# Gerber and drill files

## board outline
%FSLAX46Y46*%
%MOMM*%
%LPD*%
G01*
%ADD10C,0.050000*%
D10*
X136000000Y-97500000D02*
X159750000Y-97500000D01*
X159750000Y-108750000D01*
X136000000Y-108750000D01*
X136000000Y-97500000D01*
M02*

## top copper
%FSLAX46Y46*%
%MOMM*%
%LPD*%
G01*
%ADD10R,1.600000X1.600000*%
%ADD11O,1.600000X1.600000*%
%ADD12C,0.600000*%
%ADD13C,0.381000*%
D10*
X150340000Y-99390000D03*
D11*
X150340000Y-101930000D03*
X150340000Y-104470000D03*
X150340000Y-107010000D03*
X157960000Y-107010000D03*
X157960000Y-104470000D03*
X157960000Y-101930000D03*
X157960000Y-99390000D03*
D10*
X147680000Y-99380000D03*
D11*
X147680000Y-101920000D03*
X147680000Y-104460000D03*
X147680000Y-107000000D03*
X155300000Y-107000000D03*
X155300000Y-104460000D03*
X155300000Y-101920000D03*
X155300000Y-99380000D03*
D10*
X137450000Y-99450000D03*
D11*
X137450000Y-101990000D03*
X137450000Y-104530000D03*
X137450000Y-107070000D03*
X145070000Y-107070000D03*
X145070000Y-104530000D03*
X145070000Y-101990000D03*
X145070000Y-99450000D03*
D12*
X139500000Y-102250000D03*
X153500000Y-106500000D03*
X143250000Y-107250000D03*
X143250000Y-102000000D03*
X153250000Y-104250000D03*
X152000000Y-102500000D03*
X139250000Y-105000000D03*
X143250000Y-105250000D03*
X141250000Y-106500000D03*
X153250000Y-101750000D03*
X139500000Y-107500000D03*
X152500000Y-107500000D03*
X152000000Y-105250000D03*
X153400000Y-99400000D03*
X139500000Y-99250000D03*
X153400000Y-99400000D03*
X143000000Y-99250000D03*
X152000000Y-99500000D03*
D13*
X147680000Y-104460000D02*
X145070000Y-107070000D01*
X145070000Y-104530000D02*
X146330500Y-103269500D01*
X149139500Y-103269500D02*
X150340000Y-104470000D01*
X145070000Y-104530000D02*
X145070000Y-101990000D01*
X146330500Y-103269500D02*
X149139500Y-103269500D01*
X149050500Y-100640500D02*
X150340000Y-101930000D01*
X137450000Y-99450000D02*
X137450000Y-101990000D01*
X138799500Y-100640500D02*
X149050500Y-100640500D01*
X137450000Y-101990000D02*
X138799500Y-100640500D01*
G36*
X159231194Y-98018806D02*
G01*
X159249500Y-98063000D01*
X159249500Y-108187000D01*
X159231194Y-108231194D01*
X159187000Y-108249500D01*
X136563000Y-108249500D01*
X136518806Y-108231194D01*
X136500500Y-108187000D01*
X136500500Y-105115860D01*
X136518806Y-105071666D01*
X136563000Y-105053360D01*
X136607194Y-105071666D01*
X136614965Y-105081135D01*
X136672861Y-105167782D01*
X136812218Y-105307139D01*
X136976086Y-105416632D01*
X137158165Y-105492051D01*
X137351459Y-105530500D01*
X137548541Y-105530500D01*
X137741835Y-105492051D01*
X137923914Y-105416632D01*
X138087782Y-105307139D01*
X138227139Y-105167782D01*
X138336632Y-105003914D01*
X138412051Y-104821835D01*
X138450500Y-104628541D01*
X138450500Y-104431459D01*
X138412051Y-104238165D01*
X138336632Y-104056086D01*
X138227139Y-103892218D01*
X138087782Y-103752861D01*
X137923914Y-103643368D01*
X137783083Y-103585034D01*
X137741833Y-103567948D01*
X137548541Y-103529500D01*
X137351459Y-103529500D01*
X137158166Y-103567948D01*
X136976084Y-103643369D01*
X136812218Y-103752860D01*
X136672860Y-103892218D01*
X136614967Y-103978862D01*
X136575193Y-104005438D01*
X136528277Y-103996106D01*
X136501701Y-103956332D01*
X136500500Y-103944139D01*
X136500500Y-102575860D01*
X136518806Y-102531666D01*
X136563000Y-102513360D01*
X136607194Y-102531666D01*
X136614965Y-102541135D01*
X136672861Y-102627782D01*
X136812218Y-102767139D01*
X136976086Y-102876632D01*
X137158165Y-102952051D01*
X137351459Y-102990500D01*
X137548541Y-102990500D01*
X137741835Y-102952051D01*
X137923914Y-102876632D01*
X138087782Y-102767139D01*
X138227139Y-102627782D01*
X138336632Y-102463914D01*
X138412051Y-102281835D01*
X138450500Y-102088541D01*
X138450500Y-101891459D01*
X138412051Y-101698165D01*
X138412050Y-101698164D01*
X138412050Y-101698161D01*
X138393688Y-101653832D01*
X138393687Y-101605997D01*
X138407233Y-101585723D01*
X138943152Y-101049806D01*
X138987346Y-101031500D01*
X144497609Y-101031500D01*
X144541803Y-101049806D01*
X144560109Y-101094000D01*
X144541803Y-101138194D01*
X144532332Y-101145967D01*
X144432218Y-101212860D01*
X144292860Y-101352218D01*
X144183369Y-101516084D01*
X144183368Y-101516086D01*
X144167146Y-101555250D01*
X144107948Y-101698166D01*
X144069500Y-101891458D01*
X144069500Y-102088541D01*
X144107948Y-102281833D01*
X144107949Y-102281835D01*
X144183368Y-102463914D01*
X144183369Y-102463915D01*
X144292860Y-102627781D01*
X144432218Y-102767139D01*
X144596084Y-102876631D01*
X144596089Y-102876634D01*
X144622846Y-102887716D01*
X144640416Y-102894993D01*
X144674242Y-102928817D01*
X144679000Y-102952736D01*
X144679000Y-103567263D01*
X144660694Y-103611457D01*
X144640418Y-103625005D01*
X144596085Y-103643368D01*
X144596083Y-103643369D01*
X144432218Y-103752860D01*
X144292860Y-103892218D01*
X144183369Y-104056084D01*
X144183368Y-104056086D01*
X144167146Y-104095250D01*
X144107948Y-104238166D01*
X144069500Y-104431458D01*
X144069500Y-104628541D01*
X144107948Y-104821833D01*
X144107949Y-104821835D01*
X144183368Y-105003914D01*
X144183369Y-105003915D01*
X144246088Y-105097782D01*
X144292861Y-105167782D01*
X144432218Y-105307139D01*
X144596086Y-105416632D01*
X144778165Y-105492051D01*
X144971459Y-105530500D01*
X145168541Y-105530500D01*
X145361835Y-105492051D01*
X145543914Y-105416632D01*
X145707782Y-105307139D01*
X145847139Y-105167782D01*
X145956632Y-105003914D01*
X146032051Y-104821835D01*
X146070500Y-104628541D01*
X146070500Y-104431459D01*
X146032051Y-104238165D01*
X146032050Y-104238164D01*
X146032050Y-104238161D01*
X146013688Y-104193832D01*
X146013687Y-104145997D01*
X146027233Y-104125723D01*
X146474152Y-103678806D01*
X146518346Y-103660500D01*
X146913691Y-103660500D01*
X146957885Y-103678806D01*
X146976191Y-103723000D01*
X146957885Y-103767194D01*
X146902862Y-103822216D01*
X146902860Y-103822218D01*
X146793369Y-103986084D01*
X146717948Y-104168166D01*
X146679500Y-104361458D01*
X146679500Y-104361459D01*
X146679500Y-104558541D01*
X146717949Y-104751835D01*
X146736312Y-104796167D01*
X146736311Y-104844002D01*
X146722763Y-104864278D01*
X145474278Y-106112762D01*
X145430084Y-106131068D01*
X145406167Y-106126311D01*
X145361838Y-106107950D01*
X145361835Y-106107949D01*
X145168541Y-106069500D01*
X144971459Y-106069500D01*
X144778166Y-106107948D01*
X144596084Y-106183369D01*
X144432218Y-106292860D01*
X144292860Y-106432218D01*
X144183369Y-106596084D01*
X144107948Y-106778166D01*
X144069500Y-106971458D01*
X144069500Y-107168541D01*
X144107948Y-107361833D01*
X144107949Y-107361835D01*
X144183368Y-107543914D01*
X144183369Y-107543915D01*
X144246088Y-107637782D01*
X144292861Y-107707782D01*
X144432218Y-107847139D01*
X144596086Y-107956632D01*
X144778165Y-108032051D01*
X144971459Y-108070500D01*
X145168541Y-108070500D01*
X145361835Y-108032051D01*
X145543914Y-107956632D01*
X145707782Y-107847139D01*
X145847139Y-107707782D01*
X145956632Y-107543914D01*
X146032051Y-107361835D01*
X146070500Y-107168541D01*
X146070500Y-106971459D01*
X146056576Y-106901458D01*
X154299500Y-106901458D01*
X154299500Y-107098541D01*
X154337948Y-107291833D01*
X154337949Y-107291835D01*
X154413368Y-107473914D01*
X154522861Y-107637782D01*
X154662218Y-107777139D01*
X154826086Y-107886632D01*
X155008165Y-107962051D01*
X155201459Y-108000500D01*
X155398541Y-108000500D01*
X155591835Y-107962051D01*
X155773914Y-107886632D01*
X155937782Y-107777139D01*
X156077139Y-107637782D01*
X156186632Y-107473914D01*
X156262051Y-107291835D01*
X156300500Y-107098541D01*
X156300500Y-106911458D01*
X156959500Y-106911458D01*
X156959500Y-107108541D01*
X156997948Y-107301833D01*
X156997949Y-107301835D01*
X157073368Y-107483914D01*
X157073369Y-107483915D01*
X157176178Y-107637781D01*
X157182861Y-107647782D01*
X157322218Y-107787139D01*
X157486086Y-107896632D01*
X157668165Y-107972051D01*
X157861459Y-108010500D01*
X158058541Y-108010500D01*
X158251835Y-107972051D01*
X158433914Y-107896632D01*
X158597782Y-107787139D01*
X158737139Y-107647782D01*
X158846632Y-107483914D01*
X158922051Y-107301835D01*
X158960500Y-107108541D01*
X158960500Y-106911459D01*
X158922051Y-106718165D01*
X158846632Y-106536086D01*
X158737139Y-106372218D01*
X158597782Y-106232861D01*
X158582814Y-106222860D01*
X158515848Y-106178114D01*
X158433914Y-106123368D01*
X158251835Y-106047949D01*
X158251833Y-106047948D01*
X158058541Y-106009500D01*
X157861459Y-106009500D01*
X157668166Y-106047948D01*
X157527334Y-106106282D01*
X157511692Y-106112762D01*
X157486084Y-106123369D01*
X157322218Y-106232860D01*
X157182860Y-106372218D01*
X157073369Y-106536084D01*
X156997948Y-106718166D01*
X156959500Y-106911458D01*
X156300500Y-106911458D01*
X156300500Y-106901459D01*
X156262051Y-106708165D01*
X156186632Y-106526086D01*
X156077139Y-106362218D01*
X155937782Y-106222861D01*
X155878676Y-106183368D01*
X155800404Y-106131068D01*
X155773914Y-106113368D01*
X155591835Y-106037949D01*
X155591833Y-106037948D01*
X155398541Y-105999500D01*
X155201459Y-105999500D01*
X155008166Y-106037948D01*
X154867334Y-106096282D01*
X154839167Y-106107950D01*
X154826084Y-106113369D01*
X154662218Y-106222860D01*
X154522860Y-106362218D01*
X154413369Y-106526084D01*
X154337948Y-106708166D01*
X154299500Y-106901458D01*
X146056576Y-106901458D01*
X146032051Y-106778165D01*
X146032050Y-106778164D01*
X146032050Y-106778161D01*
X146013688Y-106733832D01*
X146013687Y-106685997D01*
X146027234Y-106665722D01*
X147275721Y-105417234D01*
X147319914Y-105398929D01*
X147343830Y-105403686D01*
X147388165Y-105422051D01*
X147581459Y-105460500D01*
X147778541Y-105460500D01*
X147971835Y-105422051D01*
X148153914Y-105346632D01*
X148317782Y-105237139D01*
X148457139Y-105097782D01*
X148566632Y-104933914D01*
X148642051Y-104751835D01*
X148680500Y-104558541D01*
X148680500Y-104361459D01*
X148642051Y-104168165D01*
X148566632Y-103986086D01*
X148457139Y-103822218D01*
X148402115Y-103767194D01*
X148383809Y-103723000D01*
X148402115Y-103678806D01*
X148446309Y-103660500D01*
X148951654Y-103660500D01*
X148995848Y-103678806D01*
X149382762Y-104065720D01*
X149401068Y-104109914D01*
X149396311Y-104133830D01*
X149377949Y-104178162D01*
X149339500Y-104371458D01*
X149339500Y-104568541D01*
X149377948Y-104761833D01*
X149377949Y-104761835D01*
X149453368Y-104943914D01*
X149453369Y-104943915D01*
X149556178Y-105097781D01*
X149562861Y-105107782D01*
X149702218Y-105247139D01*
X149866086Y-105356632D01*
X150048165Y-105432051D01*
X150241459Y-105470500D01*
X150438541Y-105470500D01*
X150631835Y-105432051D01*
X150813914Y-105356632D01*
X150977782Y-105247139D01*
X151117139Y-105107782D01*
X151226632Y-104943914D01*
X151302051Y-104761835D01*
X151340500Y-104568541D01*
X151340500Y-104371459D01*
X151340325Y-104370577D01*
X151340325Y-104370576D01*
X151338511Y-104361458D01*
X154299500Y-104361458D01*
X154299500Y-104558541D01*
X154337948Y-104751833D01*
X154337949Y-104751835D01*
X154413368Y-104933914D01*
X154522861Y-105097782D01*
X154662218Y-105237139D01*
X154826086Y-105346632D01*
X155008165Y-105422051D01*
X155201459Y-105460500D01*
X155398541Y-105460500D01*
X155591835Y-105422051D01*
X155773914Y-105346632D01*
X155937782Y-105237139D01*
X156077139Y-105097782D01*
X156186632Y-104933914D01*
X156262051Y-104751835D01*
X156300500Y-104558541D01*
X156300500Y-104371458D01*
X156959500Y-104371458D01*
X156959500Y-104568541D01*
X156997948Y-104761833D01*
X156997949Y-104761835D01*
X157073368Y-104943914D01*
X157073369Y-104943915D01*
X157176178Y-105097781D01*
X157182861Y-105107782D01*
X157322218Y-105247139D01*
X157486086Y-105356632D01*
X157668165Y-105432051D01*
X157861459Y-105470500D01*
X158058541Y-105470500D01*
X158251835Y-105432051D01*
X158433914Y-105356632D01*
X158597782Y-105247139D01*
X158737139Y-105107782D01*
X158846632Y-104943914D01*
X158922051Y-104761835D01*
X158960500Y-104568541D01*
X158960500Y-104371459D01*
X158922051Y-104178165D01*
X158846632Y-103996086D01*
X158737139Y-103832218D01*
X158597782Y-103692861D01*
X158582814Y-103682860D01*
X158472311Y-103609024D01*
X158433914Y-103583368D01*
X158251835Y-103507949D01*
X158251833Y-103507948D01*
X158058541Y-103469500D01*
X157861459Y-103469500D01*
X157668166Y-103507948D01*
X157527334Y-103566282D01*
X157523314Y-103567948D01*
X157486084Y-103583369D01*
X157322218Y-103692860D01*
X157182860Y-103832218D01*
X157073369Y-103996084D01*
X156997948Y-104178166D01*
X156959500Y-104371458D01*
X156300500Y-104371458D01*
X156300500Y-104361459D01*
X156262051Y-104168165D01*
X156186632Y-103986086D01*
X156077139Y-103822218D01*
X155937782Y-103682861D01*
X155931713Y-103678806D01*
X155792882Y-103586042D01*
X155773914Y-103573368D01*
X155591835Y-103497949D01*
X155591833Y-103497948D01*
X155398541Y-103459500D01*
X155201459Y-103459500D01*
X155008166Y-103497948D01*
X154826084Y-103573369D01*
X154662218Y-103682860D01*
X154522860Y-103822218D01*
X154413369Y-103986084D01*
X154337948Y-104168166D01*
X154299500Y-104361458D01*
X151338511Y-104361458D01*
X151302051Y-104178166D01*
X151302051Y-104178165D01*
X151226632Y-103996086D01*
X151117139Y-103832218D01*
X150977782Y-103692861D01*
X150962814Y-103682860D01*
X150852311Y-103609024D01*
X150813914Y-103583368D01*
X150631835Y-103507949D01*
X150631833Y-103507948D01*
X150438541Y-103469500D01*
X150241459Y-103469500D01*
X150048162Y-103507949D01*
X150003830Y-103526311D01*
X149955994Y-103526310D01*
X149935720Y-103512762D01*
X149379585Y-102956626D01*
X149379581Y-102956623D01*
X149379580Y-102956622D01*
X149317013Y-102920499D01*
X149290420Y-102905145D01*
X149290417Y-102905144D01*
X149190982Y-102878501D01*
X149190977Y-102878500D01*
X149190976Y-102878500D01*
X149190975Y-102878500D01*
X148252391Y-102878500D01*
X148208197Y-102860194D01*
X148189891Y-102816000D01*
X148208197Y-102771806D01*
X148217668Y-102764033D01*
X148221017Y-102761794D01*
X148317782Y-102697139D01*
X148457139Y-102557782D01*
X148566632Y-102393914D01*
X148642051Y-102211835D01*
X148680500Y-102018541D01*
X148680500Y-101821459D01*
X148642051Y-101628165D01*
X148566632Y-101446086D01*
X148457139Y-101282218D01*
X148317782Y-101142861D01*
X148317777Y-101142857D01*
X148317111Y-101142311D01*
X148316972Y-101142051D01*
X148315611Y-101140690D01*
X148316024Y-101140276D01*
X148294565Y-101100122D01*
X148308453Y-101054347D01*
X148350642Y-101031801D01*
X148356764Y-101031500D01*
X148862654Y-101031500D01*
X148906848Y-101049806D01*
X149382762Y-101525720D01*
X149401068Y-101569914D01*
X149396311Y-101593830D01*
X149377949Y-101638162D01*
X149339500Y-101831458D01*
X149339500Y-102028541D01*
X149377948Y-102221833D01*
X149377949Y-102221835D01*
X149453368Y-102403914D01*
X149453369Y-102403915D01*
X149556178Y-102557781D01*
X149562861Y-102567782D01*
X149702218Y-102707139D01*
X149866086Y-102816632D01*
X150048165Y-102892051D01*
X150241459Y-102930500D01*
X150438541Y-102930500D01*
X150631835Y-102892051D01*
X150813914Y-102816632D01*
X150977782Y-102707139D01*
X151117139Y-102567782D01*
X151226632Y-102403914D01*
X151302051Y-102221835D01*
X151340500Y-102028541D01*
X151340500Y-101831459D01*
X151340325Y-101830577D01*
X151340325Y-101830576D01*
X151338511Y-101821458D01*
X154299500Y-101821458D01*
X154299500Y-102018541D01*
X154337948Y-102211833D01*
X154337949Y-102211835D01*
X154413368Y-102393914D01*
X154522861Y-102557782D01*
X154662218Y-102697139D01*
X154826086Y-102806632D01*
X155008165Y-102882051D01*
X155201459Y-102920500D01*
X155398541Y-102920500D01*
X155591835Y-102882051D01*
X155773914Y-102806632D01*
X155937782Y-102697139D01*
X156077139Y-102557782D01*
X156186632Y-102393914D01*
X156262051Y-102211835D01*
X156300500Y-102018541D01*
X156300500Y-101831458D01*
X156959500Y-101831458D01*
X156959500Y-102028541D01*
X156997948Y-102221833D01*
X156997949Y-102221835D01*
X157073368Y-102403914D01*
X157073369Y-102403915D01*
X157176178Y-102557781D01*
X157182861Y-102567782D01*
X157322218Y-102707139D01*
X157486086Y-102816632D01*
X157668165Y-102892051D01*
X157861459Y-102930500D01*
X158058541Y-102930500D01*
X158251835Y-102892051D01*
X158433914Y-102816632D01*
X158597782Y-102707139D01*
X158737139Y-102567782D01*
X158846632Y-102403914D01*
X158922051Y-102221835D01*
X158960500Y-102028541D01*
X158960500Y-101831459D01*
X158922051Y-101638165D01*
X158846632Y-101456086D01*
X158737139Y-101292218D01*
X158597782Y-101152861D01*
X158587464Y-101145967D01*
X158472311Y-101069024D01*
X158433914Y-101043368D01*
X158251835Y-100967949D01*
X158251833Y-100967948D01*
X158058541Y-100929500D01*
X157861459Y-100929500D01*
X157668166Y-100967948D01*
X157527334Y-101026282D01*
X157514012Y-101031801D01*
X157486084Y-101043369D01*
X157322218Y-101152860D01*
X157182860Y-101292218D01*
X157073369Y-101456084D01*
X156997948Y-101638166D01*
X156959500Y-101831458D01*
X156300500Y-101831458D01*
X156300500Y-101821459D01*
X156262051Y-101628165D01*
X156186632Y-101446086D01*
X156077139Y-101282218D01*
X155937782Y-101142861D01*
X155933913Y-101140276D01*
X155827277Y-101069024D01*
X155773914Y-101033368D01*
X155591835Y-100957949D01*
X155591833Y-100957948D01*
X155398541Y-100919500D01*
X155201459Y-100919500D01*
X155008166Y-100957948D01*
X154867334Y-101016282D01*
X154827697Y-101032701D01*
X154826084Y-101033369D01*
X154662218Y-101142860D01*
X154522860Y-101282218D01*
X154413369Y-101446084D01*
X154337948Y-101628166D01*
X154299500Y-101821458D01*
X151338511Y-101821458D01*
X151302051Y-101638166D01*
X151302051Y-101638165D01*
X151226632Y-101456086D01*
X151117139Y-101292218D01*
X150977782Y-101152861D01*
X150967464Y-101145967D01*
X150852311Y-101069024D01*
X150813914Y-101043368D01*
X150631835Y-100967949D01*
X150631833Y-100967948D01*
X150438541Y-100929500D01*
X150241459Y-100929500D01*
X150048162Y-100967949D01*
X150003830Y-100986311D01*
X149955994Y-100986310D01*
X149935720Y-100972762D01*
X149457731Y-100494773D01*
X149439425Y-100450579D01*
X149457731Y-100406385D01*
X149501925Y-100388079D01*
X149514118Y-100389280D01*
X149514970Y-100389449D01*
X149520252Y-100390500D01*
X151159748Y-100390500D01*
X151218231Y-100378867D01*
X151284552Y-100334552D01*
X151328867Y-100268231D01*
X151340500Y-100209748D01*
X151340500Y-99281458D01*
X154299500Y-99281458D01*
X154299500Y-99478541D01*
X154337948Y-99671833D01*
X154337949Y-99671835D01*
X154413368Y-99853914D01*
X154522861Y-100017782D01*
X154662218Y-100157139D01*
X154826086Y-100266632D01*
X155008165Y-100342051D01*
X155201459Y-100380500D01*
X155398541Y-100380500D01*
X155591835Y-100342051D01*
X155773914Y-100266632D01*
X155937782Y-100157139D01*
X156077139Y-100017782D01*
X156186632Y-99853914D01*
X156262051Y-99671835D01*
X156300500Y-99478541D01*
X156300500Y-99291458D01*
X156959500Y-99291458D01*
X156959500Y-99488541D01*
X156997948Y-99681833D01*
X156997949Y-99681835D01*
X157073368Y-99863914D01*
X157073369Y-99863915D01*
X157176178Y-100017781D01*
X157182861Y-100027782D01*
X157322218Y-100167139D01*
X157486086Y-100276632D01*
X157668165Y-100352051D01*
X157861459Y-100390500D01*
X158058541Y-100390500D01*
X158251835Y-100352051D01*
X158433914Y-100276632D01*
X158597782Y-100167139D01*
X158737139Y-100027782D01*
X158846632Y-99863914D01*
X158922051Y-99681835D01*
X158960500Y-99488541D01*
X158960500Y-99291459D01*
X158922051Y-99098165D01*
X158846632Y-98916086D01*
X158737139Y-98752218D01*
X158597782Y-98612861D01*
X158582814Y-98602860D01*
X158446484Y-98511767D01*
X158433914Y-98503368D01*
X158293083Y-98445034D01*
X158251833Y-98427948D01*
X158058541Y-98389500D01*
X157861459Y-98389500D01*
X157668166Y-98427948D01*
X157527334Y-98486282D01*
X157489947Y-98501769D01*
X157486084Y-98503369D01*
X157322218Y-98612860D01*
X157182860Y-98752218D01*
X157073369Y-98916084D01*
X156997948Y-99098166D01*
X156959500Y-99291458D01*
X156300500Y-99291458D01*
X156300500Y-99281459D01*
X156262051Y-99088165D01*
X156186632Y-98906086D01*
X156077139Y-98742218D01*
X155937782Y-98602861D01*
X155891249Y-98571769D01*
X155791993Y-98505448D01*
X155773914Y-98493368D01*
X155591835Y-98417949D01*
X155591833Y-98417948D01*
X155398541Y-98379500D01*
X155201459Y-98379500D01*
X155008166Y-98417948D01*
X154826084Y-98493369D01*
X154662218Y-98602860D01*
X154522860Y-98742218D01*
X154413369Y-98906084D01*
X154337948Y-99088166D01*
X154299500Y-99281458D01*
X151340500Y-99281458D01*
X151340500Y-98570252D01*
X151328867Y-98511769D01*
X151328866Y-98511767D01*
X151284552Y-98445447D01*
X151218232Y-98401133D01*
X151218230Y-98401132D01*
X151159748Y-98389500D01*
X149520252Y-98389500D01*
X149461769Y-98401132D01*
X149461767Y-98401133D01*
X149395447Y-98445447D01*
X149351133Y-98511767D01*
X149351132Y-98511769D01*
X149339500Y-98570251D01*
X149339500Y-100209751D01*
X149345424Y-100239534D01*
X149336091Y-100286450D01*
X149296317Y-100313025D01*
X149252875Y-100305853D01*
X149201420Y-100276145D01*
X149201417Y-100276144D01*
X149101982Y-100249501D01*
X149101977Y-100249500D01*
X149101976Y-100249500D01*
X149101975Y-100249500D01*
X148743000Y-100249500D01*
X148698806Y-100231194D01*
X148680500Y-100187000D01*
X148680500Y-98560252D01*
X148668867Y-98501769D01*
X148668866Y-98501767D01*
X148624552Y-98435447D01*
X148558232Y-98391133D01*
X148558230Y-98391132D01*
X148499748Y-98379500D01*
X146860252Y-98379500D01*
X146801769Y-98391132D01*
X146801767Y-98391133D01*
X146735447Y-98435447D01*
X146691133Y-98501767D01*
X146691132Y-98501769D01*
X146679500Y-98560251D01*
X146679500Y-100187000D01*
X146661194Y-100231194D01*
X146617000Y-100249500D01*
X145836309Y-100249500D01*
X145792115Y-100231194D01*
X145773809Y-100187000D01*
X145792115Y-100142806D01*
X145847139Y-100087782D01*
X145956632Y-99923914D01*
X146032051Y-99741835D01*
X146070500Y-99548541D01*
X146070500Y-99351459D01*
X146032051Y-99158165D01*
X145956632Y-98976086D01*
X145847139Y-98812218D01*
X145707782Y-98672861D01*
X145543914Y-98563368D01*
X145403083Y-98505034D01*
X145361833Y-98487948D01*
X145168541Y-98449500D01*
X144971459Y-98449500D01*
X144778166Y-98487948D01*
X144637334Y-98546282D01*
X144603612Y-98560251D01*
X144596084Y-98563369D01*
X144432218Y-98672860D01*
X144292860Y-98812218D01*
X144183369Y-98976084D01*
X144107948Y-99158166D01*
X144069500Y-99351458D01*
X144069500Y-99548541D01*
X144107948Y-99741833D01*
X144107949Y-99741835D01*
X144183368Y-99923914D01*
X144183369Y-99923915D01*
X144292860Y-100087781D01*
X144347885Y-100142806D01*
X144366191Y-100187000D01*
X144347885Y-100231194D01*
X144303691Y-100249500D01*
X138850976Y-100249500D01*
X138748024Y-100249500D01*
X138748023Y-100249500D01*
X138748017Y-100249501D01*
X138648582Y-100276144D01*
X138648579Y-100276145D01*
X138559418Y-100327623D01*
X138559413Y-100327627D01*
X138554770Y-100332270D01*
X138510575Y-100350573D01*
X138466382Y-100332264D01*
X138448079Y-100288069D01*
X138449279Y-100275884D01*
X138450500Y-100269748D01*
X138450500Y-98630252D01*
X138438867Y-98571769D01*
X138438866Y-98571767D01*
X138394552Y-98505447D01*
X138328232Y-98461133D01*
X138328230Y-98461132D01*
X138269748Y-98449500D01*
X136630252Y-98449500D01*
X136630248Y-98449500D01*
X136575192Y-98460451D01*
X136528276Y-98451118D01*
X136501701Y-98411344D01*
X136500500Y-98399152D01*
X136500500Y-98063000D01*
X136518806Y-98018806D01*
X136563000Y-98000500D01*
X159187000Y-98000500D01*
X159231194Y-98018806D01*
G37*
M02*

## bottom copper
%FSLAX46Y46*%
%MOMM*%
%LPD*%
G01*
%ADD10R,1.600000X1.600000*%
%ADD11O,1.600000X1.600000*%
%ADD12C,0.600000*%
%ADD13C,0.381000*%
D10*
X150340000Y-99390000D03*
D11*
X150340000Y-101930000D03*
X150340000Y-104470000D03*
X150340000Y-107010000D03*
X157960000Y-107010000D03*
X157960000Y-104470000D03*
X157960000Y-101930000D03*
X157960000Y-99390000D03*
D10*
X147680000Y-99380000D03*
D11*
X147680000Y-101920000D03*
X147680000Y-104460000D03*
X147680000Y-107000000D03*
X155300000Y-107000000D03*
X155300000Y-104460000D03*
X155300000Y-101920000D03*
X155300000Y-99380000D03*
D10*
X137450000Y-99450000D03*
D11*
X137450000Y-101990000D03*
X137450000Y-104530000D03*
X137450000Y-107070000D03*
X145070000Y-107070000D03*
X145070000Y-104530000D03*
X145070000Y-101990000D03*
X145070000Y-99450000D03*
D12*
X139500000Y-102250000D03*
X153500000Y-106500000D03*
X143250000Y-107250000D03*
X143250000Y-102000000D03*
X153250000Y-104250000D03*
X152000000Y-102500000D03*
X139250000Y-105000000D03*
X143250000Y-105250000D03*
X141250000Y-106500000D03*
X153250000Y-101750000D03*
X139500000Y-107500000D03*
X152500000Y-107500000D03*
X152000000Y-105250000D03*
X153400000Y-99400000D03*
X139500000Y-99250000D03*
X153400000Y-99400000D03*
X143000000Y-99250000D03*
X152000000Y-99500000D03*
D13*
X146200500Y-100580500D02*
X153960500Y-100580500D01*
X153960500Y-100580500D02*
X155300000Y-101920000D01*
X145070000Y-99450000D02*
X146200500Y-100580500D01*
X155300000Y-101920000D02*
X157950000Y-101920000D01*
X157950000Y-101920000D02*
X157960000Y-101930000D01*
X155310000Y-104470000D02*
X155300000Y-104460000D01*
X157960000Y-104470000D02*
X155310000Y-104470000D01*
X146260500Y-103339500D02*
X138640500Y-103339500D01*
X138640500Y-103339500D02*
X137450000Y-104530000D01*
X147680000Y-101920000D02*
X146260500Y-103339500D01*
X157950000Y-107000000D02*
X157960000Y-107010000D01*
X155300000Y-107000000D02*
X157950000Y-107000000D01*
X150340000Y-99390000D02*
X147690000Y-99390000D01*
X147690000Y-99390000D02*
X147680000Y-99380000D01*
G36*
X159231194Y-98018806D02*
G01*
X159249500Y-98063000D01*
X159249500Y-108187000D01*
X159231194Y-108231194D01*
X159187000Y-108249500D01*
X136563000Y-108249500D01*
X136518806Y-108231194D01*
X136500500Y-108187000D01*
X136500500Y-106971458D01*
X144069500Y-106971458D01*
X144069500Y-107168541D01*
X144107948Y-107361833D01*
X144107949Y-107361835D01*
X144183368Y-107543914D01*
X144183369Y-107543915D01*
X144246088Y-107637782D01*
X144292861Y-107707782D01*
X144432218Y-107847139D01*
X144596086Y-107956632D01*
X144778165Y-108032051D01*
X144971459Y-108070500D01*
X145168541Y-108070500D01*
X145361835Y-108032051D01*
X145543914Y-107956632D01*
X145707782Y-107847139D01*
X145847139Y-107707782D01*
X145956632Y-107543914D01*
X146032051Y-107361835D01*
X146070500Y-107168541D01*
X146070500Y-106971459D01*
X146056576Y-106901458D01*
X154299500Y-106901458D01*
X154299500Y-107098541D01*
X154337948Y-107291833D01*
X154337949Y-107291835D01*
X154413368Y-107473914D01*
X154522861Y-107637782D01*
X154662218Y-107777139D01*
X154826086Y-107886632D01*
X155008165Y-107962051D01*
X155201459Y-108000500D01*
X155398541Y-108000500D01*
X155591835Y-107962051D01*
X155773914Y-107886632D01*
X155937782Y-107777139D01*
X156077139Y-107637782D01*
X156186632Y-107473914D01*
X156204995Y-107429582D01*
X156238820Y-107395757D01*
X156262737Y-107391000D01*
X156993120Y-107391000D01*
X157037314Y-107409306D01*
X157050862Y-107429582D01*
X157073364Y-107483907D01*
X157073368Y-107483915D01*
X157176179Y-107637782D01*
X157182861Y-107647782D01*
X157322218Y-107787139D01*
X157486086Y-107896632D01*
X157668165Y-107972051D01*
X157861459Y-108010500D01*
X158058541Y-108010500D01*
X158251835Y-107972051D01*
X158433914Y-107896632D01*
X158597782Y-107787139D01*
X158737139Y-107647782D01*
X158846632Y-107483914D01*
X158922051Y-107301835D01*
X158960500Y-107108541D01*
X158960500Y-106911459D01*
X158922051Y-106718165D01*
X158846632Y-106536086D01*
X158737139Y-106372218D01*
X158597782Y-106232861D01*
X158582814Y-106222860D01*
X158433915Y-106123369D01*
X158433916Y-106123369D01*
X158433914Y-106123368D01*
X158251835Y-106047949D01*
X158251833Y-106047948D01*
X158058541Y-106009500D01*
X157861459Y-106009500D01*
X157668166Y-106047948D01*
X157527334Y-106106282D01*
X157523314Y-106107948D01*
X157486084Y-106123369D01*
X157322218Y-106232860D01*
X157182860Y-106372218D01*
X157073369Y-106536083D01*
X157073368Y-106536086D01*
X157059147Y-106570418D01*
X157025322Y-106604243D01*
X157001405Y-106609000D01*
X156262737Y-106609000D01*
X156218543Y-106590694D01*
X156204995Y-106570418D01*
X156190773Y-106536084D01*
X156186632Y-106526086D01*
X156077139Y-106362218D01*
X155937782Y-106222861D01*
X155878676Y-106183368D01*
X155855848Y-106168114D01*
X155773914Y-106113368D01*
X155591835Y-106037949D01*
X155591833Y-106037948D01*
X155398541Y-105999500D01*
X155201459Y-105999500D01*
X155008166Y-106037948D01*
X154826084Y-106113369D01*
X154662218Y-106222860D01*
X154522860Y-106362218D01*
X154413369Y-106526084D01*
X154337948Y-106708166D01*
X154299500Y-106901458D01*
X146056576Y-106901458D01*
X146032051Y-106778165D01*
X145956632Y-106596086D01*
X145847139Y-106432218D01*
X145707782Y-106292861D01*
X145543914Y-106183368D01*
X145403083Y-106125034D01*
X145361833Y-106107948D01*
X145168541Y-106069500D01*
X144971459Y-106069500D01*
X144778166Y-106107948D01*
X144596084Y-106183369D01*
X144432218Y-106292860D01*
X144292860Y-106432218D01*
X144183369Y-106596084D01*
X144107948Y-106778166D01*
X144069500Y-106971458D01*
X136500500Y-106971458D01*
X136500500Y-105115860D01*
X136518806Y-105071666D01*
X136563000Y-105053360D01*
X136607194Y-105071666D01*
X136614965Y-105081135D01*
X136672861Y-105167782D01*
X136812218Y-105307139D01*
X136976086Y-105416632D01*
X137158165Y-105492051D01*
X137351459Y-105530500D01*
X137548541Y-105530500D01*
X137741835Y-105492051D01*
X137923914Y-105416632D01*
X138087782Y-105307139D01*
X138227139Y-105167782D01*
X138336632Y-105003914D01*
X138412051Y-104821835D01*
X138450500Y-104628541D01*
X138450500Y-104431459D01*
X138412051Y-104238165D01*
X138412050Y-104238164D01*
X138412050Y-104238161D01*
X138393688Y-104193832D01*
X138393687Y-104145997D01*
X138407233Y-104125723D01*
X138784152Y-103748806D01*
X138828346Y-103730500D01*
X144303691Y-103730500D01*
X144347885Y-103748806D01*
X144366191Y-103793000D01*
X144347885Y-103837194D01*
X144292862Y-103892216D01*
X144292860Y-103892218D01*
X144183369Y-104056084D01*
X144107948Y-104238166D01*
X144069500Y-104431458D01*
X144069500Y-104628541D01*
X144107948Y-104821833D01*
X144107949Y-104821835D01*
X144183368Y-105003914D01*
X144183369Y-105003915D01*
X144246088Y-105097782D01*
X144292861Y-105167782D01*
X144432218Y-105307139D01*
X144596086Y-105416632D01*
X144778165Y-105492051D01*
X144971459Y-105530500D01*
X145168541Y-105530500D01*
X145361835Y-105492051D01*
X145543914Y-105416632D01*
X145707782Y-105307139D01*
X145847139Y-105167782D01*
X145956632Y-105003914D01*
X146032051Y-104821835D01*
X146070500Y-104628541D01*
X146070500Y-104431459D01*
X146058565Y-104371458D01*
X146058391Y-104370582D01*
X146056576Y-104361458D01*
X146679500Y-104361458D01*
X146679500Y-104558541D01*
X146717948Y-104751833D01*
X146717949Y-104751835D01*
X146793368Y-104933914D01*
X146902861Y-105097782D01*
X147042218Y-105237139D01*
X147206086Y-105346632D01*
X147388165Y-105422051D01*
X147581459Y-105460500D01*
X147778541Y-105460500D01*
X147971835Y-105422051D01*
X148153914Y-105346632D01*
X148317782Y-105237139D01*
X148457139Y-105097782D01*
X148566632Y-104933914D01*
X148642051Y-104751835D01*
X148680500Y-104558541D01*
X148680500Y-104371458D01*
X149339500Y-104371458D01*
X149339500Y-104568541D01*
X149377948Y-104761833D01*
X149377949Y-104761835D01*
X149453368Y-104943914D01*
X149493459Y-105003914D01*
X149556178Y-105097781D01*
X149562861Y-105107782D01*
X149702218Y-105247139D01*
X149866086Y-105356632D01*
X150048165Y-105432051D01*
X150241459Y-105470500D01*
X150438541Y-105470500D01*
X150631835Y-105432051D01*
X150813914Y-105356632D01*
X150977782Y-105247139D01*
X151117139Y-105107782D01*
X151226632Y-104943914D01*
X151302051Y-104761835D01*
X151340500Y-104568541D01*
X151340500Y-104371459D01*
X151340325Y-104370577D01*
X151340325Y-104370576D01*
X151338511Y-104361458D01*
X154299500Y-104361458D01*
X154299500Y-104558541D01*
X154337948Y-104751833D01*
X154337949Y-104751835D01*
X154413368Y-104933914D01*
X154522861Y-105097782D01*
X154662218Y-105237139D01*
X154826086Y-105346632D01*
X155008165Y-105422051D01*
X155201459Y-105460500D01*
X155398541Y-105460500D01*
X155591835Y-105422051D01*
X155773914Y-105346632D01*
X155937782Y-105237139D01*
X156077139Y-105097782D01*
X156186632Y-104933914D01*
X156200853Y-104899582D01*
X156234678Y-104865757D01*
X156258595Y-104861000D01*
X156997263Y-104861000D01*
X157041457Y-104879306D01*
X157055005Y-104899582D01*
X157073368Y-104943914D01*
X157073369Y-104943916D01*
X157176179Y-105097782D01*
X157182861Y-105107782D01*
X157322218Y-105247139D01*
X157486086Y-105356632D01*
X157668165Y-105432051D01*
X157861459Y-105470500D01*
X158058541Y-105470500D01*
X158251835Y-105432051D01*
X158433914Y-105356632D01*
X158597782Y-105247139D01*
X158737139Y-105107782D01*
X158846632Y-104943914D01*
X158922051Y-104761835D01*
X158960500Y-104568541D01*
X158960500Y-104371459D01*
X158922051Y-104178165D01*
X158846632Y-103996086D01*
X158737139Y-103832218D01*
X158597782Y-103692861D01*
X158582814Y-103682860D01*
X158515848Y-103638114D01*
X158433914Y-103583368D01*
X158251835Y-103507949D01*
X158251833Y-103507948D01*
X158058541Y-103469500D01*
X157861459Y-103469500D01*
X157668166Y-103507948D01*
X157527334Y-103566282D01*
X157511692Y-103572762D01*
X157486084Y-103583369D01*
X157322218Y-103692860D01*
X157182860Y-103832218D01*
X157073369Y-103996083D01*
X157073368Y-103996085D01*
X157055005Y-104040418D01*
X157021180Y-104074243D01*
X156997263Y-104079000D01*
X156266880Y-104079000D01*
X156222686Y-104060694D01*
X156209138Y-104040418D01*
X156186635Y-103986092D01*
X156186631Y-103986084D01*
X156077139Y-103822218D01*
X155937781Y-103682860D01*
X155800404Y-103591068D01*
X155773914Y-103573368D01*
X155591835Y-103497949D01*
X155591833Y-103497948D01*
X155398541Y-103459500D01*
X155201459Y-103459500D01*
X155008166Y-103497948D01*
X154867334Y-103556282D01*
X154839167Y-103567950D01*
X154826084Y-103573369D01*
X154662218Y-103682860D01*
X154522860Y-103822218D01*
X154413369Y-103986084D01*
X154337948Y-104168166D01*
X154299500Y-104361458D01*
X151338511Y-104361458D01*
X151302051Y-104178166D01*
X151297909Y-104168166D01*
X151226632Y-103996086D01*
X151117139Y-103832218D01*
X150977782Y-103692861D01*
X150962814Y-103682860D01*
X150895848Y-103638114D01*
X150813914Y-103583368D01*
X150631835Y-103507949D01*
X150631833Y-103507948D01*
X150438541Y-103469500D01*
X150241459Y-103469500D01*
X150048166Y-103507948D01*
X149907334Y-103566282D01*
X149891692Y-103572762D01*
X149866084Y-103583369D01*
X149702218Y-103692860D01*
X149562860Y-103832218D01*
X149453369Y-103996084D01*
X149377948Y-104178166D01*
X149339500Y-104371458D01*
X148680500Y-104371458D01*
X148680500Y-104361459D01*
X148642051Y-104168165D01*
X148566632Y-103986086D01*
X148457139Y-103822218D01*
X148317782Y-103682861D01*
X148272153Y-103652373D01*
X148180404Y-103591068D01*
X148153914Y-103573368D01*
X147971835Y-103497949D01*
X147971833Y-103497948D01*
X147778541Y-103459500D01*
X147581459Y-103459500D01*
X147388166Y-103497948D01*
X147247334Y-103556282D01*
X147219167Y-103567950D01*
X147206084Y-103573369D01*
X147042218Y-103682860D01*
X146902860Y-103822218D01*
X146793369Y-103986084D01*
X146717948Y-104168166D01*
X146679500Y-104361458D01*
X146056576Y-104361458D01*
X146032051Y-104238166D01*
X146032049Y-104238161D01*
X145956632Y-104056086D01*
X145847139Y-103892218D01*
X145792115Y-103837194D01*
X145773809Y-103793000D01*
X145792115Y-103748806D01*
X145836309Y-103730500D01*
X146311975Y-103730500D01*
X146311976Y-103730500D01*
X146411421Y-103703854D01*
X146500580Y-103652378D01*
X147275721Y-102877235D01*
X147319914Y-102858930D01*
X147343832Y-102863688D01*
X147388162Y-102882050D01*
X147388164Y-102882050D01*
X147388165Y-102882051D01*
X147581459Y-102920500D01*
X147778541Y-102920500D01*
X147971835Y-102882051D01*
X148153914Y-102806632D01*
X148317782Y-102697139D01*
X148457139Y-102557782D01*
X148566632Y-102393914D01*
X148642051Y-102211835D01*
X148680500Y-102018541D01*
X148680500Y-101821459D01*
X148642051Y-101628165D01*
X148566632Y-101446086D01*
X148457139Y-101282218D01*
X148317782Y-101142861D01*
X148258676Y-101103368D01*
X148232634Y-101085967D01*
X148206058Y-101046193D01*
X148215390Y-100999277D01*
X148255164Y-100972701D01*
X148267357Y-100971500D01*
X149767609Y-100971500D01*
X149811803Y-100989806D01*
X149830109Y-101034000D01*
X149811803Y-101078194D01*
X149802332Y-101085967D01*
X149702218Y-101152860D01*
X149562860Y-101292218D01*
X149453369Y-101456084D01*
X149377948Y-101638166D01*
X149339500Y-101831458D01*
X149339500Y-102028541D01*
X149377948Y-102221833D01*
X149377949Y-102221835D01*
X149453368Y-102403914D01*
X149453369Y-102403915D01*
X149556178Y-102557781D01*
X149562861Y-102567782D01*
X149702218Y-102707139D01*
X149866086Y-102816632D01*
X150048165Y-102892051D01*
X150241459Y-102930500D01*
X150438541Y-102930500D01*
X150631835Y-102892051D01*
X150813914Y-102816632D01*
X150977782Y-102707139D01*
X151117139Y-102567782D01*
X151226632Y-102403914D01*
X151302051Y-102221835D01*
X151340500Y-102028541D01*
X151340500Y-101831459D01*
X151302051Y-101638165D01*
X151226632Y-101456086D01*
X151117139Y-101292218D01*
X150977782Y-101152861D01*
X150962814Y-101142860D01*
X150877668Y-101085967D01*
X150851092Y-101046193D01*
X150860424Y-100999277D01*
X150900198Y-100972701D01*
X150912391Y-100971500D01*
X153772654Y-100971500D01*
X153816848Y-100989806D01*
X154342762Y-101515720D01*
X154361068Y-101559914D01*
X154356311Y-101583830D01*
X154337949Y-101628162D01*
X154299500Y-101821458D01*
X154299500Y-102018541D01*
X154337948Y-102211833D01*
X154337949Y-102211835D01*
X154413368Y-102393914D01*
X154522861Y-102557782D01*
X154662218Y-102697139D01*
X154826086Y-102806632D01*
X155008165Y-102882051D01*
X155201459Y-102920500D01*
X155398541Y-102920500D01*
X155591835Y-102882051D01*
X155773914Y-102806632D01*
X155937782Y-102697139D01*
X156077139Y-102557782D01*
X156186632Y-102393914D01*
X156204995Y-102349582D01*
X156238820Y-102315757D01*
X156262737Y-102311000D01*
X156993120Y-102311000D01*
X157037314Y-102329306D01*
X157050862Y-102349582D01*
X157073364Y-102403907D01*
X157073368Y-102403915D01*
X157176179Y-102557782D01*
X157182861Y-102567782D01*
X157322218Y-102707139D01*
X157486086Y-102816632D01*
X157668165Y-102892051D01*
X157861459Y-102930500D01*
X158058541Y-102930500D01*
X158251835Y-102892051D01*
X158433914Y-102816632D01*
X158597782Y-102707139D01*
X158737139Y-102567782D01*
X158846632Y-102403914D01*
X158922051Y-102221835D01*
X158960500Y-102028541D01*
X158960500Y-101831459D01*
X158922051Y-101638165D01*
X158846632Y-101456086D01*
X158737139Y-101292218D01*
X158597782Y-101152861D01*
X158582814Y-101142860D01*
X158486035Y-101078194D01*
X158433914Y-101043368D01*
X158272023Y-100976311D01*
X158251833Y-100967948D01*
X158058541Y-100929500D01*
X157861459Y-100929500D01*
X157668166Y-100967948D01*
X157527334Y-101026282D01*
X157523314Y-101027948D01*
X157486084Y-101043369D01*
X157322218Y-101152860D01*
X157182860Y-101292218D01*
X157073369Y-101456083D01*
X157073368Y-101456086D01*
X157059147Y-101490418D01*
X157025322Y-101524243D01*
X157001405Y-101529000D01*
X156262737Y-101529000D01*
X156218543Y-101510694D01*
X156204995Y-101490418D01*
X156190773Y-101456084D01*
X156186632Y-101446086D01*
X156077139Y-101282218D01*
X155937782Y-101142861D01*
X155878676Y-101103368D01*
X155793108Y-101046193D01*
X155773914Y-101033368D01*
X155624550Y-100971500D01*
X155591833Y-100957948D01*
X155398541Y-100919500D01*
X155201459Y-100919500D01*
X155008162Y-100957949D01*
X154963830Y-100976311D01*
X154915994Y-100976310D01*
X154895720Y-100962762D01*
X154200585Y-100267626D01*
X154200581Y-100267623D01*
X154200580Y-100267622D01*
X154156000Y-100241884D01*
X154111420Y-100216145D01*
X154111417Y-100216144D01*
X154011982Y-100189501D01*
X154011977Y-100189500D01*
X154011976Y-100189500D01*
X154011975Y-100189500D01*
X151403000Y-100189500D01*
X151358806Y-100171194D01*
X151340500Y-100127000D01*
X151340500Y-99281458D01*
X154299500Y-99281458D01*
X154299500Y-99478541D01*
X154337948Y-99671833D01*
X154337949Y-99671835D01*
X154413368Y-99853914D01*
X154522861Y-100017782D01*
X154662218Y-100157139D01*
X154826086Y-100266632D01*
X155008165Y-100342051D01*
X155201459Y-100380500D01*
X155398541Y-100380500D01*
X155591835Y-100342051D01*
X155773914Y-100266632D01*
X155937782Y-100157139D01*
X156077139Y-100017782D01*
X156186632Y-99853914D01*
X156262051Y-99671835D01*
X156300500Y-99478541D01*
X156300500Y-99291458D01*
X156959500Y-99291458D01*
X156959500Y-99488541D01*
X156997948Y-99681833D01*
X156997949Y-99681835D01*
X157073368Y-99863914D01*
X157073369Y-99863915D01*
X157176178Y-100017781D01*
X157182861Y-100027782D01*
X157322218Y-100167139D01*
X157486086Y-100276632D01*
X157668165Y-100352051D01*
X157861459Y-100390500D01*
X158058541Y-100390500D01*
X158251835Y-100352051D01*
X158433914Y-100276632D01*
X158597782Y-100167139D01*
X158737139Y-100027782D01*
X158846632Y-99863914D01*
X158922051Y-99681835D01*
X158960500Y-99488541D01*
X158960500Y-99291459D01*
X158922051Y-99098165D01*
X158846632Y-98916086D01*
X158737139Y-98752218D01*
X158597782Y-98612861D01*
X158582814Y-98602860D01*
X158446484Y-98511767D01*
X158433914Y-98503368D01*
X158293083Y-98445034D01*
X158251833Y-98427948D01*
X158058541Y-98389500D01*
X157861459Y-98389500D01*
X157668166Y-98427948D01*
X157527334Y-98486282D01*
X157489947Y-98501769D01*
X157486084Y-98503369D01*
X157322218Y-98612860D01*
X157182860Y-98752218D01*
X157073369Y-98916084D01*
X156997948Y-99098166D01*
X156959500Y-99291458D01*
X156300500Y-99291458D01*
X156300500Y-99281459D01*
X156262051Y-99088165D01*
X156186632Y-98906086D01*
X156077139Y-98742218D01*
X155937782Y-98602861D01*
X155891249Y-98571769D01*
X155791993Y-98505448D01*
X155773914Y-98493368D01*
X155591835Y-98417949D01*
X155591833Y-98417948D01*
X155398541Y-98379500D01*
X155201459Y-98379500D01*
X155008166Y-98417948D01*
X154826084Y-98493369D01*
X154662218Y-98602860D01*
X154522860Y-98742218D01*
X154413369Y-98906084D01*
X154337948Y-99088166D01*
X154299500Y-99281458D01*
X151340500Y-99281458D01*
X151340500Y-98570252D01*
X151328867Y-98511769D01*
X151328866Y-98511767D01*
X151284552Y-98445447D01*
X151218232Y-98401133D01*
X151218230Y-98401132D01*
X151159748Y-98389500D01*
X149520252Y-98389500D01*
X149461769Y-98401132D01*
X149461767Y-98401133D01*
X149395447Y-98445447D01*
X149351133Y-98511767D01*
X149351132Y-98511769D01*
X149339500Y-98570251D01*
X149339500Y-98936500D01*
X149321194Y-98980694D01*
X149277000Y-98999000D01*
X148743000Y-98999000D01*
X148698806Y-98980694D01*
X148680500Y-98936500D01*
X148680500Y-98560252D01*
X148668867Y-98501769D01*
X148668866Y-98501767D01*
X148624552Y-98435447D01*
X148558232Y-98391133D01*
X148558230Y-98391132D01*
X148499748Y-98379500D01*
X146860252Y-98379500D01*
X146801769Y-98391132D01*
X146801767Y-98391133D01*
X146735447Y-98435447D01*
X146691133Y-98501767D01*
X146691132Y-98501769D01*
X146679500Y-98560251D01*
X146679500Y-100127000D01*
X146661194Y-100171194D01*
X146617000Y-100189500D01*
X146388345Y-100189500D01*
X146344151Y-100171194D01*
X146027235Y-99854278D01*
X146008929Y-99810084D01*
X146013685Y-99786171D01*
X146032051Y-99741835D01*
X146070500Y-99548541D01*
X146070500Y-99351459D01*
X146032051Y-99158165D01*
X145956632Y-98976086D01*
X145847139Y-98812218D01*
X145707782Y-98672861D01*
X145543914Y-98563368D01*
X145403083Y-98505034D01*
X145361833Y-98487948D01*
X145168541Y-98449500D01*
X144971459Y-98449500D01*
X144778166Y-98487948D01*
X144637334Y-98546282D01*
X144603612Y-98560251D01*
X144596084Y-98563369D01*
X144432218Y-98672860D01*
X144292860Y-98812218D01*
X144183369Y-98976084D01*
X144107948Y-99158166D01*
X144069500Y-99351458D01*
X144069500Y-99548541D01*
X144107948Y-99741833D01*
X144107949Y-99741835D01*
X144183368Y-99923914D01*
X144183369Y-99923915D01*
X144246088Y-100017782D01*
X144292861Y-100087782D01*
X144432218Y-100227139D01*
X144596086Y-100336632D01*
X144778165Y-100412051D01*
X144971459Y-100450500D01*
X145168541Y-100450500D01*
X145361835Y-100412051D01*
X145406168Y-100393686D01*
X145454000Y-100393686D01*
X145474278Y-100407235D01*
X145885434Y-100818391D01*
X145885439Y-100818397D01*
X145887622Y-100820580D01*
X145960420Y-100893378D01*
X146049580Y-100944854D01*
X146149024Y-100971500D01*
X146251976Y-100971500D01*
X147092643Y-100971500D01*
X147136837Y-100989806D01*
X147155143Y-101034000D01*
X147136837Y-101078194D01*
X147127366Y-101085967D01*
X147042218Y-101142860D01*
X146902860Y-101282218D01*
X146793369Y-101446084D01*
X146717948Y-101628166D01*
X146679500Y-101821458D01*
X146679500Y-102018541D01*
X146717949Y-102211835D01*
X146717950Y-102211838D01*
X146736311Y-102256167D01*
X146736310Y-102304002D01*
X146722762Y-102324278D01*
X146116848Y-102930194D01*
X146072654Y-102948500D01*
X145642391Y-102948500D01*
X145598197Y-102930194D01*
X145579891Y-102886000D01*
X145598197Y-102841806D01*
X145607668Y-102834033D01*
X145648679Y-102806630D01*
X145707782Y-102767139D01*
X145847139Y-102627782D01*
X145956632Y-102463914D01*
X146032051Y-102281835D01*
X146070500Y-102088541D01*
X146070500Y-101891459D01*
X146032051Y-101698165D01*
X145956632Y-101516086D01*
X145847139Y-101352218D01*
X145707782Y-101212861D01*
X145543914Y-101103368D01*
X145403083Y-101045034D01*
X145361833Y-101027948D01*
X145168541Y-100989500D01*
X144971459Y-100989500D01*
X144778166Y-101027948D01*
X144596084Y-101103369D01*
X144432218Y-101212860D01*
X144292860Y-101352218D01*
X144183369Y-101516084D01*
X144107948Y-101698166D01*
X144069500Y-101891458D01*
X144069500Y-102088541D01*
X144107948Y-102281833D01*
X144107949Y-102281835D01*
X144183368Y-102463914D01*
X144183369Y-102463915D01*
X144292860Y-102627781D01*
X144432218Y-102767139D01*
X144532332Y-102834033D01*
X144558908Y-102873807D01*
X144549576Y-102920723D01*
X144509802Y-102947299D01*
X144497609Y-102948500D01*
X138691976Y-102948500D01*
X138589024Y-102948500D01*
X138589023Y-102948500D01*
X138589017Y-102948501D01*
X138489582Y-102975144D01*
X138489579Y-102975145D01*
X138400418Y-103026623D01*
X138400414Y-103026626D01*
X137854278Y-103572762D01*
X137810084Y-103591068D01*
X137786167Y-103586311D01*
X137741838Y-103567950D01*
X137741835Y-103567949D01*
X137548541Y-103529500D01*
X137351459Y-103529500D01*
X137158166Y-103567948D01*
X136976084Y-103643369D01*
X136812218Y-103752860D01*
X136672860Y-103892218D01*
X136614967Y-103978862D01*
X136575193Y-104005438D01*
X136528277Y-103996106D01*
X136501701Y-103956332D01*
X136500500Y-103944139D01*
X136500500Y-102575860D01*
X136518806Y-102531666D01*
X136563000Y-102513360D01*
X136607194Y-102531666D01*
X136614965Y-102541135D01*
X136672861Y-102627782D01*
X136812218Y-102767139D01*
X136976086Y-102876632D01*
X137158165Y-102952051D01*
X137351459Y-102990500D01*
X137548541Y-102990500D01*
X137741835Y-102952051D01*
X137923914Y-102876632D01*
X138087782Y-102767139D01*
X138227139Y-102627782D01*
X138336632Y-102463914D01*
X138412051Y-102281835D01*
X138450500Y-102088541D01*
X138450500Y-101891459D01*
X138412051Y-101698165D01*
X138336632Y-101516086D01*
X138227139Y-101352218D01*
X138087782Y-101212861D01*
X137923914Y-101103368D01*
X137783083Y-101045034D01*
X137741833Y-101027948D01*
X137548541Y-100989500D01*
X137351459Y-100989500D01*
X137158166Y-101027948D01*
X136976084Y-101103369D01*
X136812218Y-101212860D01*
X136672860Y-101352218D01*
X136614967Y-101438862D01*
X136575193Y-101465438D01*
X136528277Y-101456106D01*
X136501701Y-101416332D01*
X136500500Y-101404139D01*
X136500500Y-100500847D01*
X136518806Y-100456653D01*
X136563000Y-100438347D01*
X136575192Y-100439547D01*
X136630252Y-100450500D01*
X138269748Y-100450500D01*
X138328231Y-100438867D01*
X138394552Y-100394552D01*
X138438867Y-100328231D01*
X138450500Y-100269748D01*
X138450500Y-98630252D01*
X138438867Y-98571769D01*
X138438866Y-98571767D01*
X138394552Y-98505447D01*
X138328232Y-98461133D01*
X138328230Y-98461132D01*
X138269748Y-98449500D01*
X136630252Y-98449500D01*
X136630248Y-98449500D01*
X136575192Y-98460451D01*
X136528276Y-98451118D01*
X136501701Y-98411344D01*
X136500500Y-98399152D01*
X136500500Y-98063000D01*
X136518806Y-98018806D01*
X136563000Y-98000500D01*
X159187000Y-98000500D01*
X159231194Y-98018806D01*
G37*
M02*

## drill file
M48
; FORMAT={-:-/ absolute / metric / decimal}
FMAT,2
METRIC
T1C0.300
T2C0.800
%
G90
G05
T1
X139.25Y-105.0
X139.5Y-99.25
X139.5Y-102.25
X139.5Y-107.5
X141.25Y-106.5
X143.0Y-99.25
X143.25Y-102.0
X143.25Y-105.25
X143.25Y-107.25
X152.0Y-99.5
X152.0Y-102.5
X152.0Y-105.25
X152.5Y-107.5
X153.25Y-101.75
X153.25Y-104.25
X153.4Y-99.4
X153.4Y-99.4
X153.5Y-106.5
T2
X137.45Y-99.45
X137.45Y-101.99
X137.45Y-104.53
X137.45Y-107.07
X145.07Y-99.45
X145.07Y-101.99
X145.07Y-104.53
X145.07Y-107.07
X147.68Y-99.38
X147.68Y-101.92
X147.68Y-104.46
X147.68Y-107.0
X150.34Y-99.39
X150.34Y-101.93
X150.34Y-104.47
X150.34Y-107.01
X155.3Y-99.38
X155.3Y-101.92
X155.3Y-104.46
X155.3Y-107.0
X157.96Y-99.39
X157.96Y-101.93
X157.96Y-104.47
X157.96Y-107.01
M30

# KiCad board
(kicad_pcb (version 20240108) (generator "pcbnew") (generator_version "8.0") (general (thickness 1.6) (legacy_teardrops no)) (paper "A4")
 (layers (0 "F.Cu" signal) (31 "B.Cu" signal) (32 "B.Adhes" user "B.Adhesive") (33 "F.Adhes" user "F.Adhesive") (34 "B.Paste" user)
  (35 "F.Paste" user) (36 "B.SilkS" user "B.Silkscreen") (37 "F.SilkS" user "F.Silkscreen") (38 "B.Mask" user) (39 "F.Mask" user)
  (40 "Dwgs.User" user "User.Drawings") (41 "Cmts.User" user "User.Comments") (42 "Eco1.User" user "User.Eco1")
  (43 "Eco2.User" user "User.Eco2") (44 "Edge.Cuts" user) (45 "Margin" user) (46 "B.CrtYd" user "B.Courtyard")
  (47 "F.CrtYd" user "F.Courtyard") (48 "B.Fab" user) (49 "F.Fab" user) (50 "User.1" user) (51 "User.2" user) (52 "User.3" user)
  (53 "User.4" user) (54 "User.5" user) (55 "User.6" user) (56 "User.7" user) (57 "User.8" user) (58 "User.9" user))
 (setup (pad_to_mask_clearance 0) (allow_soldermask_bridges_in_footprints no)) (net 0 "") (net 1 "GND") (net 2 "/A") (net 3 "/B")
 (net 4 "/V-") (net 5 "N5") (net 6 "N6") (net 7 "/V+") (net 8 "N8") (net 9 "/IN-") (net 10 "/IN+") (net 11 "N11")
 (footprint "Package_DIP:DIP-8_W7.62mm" (layer "F.Cu") (at 150.34 99.39)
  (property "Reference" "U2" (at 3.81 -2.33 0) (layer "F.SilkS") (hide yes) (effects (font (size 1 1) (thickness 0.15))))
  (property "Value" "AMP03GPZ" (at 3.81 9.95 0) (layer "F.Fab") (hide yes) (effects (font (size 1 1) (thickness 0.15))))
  (pad "1" thru_hole rect (at 0 0) (size 1.6 1.6) (drill 0.8) (layers "*.Cu" "*.Mask") (remove_unused_layers no) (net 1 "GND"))
  (pad "2" thru_hole oval (at 0 2.54) (size 1.6 1.6) (drill 0.8) (layers "*.Cu" "*.Mask") (remove_unused_layers no) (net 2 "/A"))
  (pad "3" thru_hole oval (at 0 5.08) (size 1.6 1.6) (drill 0.8) (layers "*.Cu" "*.Mask") (remove_unused_layers no) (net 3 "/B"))
  (pad "4" thru_hole oval (at 0 7.62) (size 1.6 1.6) (drill 0.8) (layers "*.Cu" "*.Mask") (remove_unused_layers no) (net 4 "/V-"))
  (pad "5" thru_hole oval (at 7.62 7.62) (size 1.6 1.6) (drill 0.8) (layers "*.Cu" "*.Mask") (remove_unused_layers no) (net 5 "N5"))
  (pad "6" thru_hole oval (at 7.62 5.08) (size 1.6 1.6) (drill 0.8) (layers "*.Cu" "*.Mask") (remove_unused_layers no) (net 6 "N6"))
  (pad "7" thru_hole oval (at 7.62 2.54) (size 1.6 1.6) (drill 0.8) (layers "*.Cu" "*.Mask") (remove_unused_layers no) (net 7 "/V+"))
  (pad "8" thru_hole oval (at 7.62 0) (size 1.6 1.6) (drill 0.8) (layers "*.Cu" "*.Mask") (remove_unused_layers no) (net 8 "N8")))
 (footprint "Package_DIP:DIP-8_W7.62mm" (layer "F.Cu") (at 147.68 99.38)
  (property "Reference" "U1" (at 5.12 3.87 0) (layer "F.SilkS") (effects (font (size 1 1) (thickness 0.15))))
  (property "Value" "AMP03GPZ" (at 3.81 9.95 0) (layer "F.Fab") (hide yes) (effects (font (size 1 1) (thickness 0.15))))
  (pad "1" thru_hole rect (at 0 0) (size 1.6 1.6) (drill 0.8) (layers "*.Cu" "*.Mask") (remove_unused_layers no) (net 1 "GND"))
  (pad "2" thru_hole oval (at 0 2.54) (size 1.6 1.6) (drill 0.8) (layers "*.Cu" "*.Mask") (remove_unused_layers no) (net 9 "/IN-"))
  (pad "3" thru_hole oval (at 0 5.08) (size 1.6 1.6) (drill 0.8) (layers "*.Cu" "*.Mask") (remove_unused_layers no) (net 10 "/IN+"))
  (pad "4" thru_hole oval (at 0 7.62) (size 1.6 1.6) (drill 0.8) (layers "*.Cu" "*.Mask") (remove_unused_layers no) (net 4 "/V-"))
  (pad "5" thru_hole oval (at 7.62 7.62) (size 1.6 1.6) (drill 0.8) (layers "*.Cu" "*.Mask") (remove_unused_layers no) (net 5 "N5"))
  (pad "6" thru_hole oval (at 7.62 5.08) (size 1.6 1.6) (drill 0.8) (layers "*.Cu" "*.Mask") (remove_unused_layers no) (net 6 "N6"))
  (pad "7" thru_hole oval (at 7.62 2.54) (size 1.6 1.6) (drill 0.8) (layers "*.Cu" "*.Mask") (remove_unused_layers no) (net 7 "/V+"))
  (pad "8" thru_hole oval (at 7.62 0) (size 1.6 1.6) (drill 0.8) (layers "*.Cu" "*.Mask") (remove_unused_layers no) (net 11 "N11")))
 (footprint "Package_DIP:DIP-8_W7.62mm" (layer "F.Cu") (at 137.45 99.45)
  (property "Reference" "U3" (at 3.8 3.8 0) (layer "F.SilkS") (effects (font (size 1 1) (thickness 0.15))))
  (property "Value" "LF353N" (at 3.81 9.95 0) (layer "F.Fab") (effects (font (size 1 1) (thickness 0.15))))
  (pad "1" thru_hole rect (at 0 0) (size 1.6 1.6) (drill 0.8) (layers "*.Cu" "*.Mask") (remove_unused_layers no) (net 2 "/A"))
  (pad "2" thru_hole oval (at 0 2.54) (size 1.6 1.6) (drill 0.8) (layers "*.Cu" "*.Mask") (remove_unused_layers no) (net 2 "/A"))
  (pad "3" thru_hole oval (at 0 5.08) (size 1.6 1.6) (drill 0.8) (layers "*.Cu" "*.Mask") (remove_unused_layers no) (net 9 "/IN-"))
  (pad "4" thru_hole oval (at 0 7.62) (size 1.6 1.6) (drill 0.8) (layers "*.Cu" "*.Mask") (remove_unused_layers no) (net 4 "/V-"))
  (pad "5" thru_hole oval (at 7.62 7.62) (size 1.6 1.6) (drill 0.8) (layers "*.Cu" "*.Mask") (remove_unused_layers no) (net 10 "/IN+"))
  (pad "6" thru_hole oval (at 7.62 5.08) (size 1.6 1.6) (drill 0.8) (layers "*.Cu" "*.Mask") (remove_unused_layers no) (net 3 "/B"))
  (pad "7" thru_hole oval (at 7.62 2.54) (size 1.6 1.6) (drill 0.8) (layers "*.Cu" "*.Mask") (remove_unused_layers no) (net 3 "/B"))
  (pad "8" thru_hole oval (at 7.62 0) (size 1.6 1.6) (drill 0.8) (layers "*.Cu" "*.Mask") (remove_unused_layers no) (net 7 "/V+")))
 (gr_rect (start 136 97.5) (end 159.75 108.75) (stroke (width 0.05) (type default)) (fill none) (layer "Edge.Cuts"))
 (via (at 139.5 102.25) (size 0.6) (drill 0.3) (layers "F.Cu" "B.Cu") (free yes) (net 4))
 (via (at 153.5 106.5) (size 0.6) (drill 0.3) (layers "F.Cu" "B.Cu") (free yes) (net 4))
 (via (at 143.25 107.25) (size 0.6) (drill 0.3) (layers "F.Cu" "B.Cu") (free yes) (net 4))
 (via (at 143.25 102) (size 0.6) (drill 0.3) (layers "F.Cu" "B.Cu") (free yes) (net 4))
 (via (at 153.25 104.25) (size 0.6) (drill 0.3) (layers "F.Cu" "B.Cu") (free yes) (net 4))
 (via (at 152 102.5) (size 0.6) (drill 0.3) (layers "F.Cu" "B.Cu") (free yes) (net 4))
 (via (at 139.25 105) (size 0.6) (drill 0.3) (layers "F.Cu" "B.Cu") (free yes) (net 4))
 (via (at 143.25 105.25) (size 0.6) (drill 0.3) (layers "F.Cu" "B.Cu") (free yes) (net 4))
 (via (at 141.25 106.5) (size 0.6) (drill 0.3) (layers "F.Cu" "B.Cu") (free yes) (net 4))
 (via (at 153.25 101.75) (size 0.6) (drill 0.3) (layers "F.Cu" "B.Cu") (free yes) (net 4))
 (via (at 139.5 107.5) (size 0.6) (drill 0.3) (layers "F.Cu" "B.Cu") (free yes) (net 4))
 (via (at 152.5 107.5) (size 0.6) (drill 0.3) (layers "F.Cu" "B.Cu") (free yes) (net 4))
 (via (at 152 105.25) (size 0.6) (drill 0.3) (layers "F.Cu" "B.Cu") (free yes) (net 4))
 (via (at 153.4 99.4) (size 0.6) (drill 0.3) (layers "F.Cu" "B.Cu") (free yes) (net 4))
 (via (at 139.5 99.25) (size 0.6) (drill 0.3) (layers "F.Cu" "B.Cu") (free yes) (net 4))
 (via (at 153.4 99.4) (size 0.6) (drill 0.3) (layers "F.Cu" "B.Cu") (free yes) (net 4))
 (via (at 143 99.25) (size 0.6) (drill 0.3) (layers "F.Cu" "B.Cu") (free yes) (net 4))
 (via (at 152 99.5) (size 0.6) (drill 0.3) (layers "F.Cu" "B.Cu") (free yes) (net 4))
 (segment (start 146.2005 100.5805) (end 153.9605 100.5805) (width 0.381) (layer "B.Cu") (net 7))
 (segment (start 153.9605 100.5805) (end 155.3 101.92) (width 0.381) (layer "B.Cu") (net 7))
 (segment (start 145.07 99.45) (end 146.2005 100.5805) (width 0.381) (layer "B.Cu") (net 7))
 (segment (start 155.3 101.92) (end 157.95 101.92) (width 0.381) (layer "B.Cu") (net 7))
 (segment (start 157.95 101.92) (end 157.96 101.93) (width 0.381) (layer "B.Cu") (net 7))
 (segment (start 147.68 104.46) (end 145.07 107.07) (width 0.381) (layer "F.Cu") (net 10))
 (segment (start 155.31 104.47) (end 155.3 104.46) (width 0.381) (layer "B.Cu") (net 6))
 (segment (start 157.96 104.47) (end 155.31 104.47) (width 0.381) (layer "B.Cu") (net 6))
 (segment (start 146.2605 103.3395) (end 138.6405 103.3395) (width 0.381) (layer "B.Cu") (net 9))
 (segment (start 138.6405 103.3395) (end 137.45 104.53) (width 0.381) (layer "B.Cu") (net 9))
 (segment (start 147.68 101.92) (end 146.2605 103.3395) (width 0.381) (layer "B.Cu") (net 9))
 (segment (start 157.95 107) (end 157.96 107.01) (width 0.381) (layer "B.Cu") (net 5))
 (segment (start 155.3 107) (end 157.95 107) (width 0.381) (layer "B.Cu") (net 5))
 (segment (start 145.07 104.53) (end 146.3305 103.2695) (width 0.381) (layer "F.Cu") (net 3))
 (segment (start 149.1395 103.2695) (end 150.34 104.47) (width 0.381) (layer "F.Cu") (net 3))
 (segment (start 145.07 104.53) (end 145.07 101.99) (width 0.381) (layer "F.Cu") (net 3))
 (segment (start 146.3305 103.2695) (end 149.1395 103.2695) (width 0.381) (layer "F.Cu") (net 3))
 (segment (start 149.0505 100.6405) (end 150.34 101.93) (width 0.381) (layer "F.Cu") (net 2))
 (segment (start 137.45 99.45) (end 137.45 101.99) (width 0.381) (layer "F.Cu") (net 2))
 (segment (start 138.7995 100.6405) (end 149.0505 100.6405) (width 0.381) (layer "F.Cu") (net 2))
 (segment (start 137.45 101.99) (end 138.7995 100.6405) (width 0.381) (layer "F.Cu") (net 2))
 (segment (start 150.34 99.39) (end 147.69 99.39) (width 0.381) (layer "B.Cu") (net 1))
 (segment (start 147.69 99.39) (end 147.68 99.38) (width 0.381) (layer "B.Cu") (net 1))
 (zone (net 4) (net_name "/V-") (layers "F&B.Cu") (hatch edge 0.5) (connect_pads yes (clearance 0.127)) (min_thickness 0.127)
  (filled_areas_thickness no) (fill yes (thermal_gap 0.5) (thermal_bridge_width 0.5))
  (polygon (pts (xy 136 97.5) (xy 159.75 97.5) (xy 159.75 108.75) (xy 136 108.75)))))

